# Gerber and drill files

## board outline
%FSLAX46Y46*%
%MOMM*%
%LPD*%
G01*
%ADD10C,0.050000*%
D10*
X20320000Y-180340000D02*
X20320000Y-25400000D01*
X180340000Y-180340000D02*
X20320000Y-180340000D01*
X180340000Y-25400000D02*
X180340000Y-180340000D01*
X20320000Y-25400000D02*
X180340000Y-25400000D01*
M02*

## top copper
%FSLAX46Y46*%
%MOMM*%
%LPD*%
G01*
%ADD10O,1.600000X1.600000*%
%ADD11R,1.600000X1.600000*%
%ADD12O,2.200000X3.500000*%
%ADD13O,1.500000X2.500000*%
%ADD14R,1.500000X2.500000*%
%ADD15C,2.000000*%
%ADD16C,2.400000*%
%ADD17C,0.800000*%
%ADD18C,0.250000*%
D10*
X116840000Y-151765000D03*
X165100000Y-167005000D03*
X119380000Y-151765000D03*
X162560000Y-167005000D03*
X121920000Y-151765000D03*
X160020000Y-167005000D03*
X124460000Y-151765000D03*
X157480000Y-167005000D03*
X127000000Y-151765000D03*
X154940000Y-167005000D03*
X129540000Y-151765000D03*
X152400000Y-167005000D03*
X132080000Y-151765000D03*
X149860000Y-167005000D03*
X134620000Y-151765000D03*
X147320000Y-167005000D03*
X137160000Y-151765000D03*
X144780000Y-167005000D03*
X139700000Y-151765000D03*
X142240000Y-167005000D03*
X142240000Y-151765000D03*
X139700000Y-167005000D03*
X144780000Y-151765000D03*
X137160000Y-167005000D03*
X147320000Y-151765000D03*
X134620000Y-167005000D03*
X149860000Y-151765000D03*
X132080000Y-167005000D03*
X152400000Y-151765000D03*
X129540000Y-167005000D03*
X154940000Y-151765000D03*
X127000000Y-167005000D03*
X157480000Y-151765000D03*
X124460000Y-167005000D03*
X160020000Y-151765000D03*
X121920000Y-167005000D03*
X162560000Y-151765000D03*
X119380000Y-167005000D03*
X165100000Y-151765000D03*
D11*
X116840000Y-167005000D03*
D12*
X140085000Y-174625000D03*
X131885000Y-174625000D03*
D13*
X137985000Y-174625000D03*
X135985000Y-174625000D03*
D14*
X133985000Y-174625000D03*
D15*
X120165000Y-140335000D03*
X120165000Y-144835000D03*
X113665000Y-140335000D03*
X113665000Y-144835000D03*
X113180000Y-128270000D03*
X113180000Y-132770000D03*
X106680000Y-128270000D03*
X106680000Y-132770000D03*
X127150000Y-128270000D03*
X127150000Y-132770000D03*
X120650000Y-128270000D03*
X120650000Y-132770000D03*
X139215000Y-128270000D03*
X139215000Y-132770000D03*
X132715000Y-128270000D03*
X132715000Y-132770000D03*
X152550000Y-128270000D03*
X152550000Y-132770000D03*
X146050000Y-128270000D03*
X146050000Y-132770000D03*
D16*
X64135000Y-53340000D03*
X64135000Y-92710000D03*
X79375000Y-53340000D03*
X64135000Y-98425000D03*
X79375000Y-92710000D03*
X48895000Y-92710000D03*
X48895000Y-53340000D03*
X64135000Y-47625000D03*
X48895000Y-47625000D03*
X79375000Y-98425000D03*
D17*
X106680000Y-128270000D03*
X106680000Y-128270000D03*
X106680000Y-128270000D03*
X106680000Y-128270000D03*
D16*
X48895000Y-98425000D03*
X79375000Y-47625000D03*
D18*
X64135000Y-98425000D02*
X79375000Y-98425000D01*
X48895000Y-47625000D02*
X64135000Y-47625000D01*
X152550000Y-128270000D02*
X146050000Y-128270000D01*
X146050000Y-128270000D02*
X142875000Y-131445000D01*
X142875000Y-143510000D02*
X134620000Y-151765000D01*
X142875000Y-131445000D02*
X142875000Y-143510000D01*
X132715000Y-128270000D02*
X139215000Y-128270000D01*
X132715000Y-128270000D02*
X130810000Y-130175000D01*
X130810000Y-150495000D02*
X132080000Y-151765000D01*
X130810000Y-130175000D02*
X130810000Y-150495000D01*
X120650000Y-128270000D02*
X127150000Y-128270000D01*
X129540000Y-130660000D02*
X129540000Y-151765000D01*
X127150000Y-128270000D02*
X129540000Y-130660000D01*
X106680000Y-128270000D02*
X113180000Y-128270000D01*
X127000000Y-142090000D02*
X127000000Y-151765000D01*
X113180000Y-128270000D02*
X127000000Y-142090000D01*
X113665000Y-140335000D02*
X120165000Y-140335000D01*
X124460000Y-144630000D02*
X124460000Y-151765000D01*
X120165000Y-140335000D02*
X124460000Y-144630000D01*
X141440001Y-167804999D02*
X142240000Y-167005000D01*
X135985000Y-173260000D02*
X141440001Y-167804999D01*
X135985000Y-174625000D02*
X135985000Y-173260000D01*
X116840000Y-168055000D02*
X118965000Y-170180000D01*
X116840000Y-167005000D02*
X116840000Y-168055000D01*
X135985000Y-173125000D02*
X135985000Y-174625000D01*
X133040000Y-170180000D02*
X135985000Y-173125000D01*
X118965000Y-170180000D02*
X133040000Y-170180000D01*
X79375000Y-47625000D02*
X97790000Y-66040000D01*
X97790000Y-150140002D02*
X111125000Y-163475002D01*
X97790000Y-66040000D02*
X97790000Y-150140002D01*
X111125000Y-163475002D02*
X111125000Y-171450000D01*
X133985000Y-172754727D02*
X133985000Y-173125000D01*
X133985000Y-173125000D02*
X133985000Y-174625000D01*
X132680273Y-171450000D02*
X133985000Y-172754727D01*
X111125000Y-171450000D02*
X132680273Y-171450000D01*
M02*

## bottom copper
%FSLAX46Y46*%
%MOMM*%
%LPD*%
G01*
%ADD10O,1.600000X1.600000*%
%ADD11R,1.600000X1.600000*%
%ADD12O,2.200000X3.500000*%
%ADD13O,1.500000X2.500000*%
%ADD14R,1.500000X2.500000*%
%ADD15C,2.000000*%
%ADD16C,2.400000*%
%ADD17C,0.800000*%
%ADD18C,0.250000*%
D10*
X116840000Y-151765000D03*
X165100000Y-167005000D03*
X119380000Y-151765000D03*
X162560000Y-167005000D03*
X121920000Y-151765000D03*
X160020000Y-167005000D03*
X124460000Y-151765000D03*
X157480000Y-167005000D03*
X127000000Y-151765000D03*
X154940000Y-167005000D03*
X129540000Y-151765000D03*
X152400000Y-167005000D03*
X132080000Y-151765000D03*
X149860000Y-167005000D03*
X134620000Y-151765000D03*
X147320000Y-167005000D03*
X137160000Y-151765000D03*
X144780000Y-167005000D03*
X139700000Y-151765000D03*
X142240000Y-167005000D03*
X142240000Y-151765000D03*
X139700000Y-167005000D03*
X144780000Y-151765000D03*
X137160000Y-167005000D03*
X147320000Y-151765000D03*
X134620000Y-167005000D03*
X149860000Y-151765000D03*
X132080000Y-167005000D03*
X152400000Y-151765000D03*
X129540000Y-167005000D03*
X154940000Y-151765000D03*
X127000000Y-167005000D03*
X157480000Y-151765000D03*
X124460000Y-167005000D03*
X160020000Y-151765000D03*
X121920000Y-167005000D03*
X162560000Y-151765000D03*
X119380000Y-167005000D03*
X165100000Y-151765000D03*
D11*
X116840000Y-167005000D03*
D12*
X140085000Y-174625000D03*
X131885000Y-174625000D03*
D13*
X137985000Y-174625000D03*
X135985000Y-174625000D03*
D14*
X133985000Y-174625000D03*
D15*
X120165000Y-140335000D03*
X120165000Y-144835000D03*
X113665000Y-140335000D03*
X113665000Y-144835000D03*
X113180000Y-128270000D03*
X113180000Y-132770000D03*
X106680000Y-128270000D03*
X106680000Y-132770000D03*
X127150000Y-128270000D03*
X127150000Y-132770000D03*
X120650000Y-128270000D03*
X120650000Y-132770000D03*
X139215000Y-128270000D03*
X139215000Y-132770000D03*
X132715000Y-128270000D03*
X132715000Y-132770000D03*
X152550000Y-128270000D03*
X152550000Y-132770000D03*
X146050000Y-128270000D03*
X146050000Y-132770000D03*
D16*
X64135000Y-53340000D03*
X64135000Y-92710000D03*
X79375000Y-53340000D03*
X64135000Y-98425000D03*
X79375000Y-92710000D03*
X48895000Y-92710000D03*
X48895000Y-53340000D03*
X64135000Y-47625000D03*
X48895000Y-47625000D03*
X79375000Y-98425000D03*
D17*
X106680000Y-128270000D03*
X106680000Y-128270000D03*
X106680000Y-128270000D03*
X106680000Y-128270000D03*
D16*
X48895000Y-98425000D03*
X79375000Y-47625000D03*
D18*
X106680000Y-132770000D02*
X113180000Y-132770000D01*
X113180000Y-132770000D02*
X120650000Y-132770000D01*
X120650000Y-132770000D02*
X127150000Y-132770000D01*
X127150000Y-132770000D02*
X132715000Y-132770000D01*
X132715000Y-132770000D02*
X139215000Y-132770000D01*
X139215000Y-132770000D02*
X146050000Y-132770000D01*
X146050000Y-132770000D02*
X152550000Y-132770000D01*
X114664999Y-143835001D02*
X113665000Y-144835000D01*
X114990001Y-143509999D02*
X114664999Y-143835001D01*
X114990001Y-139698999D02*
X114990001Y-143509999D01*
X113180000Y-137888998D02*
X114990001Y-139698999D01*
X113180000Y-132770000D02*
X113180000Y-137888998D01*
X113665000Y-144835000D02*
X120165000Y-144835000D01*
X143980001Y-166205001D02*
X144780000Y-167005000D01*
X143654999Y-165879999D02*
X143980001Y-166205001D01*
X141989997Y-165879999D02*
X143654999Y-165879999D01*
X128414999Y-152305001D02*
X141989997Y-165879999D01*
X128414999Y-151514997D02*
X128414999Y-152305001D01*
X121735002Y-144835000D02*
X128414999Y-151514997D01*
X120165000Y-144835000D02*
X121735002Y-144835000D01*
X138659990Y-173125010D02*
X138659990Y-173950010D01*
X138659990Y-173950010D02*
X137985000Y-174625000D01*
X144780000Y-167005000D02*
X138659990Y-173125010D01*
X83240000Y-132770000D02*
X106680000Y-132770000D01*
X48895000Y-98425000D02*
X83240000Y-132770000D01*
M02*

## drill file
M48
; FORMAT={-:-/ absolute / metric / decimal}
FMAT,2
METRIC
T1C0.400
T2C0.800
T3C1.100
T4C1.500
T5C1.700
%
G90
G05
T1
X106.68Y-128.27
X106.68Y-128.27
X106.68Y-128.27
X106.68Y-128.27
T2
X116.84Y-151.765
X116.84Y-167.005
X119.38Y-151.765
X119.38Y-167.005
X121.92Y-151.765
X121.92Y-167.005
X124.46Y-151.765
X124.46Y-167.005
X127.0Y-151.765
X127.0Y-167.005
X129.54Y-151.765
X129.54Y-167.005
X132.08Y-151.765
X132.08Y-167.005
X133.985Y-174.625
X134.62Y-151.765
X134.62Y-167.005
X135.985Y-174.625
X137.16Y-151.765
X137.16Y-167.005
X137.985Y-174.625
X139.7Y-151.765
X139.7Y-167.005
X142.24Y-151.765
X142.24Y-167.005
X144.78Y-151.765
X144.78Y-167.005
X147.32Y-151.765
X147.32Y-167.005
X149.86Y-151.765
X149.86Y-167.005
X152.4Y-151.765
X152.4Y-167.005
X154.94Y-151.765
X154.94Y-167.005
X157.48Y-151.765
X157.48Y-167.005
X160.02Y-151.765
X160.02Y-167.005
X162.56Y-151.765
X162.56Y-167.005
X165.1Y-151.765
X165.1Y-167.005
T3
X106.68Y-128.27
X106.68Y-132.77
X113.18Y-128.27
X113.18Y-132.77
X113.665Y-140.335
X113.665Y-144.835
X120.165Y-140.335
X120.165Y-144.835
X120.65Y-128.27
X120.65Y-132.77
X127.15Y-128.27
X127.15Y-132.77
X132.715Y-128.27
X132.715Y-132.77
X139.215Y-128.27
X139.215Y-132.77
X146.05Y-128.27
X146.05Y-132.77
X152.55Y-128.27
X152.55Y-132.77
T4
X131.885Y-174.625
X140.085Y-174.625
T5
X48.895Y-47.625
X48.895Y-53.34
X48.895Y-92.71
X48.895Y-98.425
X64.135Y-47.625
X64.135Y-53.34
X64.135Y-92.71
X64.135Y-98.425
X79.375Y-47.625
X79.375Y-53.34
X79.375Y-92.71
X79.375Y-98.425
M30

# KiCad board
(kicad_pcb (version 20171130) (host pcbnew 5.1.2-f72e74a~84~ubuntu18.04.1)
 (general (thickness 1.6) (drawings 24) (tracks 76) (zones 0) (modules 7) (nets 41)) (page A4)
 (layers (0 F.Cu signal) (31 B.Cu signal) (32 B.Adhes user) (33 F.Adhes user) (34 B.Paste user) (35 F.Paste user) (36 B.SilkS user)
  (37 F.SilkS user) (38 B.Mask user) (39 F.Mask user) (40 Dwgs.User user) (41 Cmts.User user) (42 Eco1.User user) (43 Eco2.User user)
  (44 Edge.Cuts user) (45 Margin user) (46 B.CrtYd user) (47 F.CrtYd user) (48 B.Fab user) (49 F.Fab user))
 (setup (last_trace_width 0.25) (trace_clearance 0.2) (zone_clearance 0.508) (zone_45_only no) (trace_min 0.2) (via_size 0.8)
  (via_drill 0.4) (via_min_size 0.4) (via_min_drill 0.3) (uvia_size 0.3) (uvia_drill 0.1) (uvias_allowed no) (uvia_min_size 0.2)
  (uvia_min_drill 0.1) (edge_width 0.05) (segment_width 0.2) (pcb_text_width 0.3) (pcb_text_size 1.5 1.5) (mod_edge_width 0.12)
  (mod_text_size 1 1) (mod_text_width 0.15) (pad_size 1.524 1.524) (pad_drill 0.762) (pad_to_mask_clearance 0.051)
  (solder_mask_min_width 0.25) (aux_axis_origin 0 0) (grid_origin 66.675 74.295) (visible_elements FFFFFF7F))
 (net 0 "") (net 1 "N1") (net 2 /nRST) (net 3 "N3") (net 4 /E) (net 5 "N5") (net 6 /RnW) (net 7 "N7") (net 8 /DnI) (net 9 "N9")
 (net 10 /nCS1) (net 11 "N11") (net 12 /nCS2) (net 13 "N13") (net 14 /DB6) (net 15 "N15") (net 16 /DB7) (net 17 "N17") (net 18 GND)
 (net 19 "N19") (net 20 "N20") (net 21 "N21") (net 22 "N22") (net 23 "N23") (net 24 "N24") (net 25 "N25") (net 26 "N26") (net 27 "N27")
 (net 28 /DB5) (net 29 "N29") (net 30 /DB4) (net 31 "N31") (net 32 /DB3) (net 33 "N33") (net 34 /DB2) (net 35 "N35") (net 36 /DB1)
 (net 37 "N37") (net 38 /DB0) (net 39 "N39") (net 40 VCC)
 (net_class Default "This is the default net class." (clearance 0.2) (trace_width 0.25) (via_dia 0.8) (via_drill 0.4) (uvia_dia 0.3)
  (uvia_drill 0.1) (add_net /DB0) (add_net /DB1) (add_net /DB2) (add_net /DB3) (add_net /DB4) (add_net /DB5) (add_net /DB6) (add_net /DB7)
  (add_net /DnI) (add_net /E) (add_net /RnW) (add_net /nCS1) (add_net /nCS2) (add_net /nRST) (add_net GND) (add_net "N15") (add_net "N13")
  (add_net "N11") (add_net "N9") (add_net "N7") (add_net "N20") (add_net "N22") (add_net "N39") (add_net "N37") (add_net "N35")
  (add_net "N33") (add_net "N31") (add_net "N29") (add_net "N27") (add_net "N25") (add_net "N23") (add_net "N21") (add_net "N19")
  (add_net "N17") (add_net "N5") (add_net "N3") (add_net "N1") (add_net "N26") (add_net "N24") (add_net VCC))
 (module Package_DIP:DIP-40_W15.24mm (layer F.Cu) (at 116.84 167.005 90)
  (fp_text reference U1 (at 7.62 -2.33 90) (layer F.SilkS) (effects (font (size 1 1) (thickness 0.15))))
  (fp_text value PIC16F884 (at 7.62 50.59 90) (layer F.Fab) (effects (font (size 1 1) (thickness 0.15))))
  (pad 40 thru_hole oval (at 15.24 0 90) (size 1.6 1.6) (drill 0.8) (layers *.Cu *.Mask) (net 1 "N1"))
  (pad 20 thru_hole oval (at 0 48.26 90) (size 1.6 1.6) (drill 0.8) (layers *.Cu *.Mask) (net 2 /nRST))
  (pad 39 thru_hole oval (at 15.24 2.54 90) (size 1.6 1.6) (drill 0.8) (layers *.Cu *.Mask) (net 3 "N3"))
  (pad 19 thru_hole oval (at 0 45.72 90) (size 1.6 1.6) (drill 0.8) (layers *.Cu *.Mask) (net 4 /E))
  (pad 38 thru_hole oval (at 15.24 5.08 90) (size 1.6 1.6) (drill 0.8) (layers *.Cu *.Mask) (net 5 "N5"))
  (pad 18 thru_hole oval (at 0 43.18 90) (size 1.6 1.6) (drill 0.8) (layers *.Cu *.Mask) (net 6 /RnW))
  (pad 37 thru_hole oval (at 15.24 7.62 90) (size 1.6 1.6) (drill 0.8) (layers *.Cu *.Mask) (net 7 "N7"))
  (pad 17 thru_hole oval (at 0 40.64 90) (size 1.6 1.6) (drill 0.8) (layers *.Cu *.Mask) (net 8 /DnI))
  (pad 36 thru_hole oval (at 15.24 10.16 90) (size 1.6 1.6) (drill 0.8) (layers *.Cu *.Mask) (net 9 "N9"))
  (pad 16 thru_hole oval (at 0 38.1 90) (size 1.6 1.6) (drill 0.8) (layers *.Cu *.Mask) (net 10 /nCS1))
  (pad 35 thru_hole oval (at 15.24 12.7 90) (size 1.6 1.6) (drill 0.8) (layers *.Cu *.Mask) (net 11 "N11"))
  (pad 15 thru_hole oval (at 0 35.56 90) (size 1.6 1.6) (drill 0.8) (layers *.Cu *.Mask) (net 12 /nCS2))
  (pad 34 thru_hole oval (at 15.24 15.24 90) (size 1.6 1.6) (drill 0.8) (layers *.Cu *.Mask) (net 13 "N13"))
  (pad 14 thru_hole oval (at 0 33.02 90) (size 1.6 1.6) (drill 0.8) (layers *.Cu *.Mask) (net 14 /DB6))
  (pad 33 thru_hole oval (at 15.24 17.78 90) (size 1.6 1.6) (drill 0.8) (layers *.Cu *.Mask) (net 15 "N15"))
  (pad 13 thru_hole oval (at 0 30.48 90) (size 1.6 1.6) (drill 0.8) (layers *.Cu *.Mask) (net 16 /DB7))
  (pad 32 thru_hole oval (at 15.24 20.32 90) (size 1.6 1.6) (drill 0.8) (layers *.Cu *.Mask) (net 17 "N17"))
  (pad 12 thru_hole oval (at 0 27.94 90) (size 1.6 1.6) (drill 0.8) (layers *.Cu *.Mask) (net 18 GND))
  (pad 31 thru_hole oval (at 15.24 22.86 90) (size 1.6 1.6) (drill 0.8) (layers *.Cu *.Mask) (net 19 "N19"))
  (pad 11 thru_hole oval (at 0 25.4 90) (size 1.6 1.6) (drill 0.8) (layers *.Cu *.Mask) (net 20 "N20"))
  (pad 30 thru_hole oval (at 15.24 25.4 90) (size 1.6 1.6) (drill 0.8) (layers *.Cu *.Mask) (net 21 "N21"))
  (pad 10 thru_hole oval (at 0 22.86 90) (size 1.6 1.6) (drill 0.8) (layers *.Cu *.Mask) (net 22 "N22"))
  (pad 29 thru_hole oval (at 15.24 27.94 90) (size 1.6 1.6) (drill 0.8) (layers *.Cu *.Mask) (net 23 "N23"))
  (pad 9 thru_hole oval (at 0 20.32 90) (size 1.6 1.6) (drill 0.8) (layers *.Cu *.Mask) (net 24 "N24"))
  (pad 28 thru_hole oval (at 15.24 30.48 90) (size 1.6 1.6) (drill 0.8) (layers *.Cu *.Mask) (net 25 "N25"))
  (pad 8 thru_hole oval (at 0 17.78 90) (size 1.6 1.6) (drill 0.8) (layers *.Cu *.Mask) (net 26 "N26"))
  (pad 27 thru_hole oval (at 15.24 33.02 90) (size 1.6 1.6) (drill 0.8) (layers *.Cu *.Mask) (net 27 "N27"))
  (pad 7 thru_hole oval (at 0 15.24 90) (size 1.6 1.6) (drill 0.8) (layers *.Cu *.Mask) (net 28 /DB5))
  (pad 26 thru_hole oval (at 15.24 35.56 90) (size 1.6 1.6) (drill 0.8) (layers *.Cu *.Mask) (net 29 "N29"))
  (pad 6 thru_hole oval (at 0 12.7 90) (size 1.6 1.6) (drill 0.8) (layers *.Cu *.Mask) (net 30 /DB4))
  (pad 25 thru_hole oval (at 15.24 38.1 90) (size 1.6 1.6) (drill 0.8) (layers *.Cu *.Mask) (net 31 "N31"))
  (pad 5 thru_hole oval (at 0 10.16 90) (size 1.6 1.6) (drill 0.8) (layers *.Cu *.Mask) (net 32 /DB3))
  (pad 24 thru_hole oval (at 15.24 40.64 90) (size 1.6 1.6) (drill 0.8) (layers *.Cu *.Mask) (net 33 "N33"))
  (pad 4 thru_hole oval (at 0 7.62 90) (size 1.6 1.6) (drill 0.8) (layers *.Cu *.Mask) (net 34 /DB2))
  (pad 23 thru_hole oval (at 15.24 43.18 90) (size 1.6 1.6) (drill 0.8) (layers *.Cu *.Mask) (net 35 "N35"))
  (pad 3 thru_hole oval (at 0 5.08 90) (size 1.6 1.6) (drill 0.8) (layers *.Cu *.Mask) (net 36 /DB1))
  (pad 22 thru_hole oval (at 15.24 45.72 90) (size 1.6 1.6) (drill 0.8) (layers *.Cu *.Mask) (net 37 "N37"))
  (pad 2 thru_hole oval (at 0 2.54 90) (size 1.6 1.6) (drill 0.8) (layers *.Cu *.Mask) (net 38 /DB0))
  (pad 21 thru_hole oval (at 15.24 48.26 90) (size 1.6 1.6) (drill 0.8) (layers *.Cu *.Mask) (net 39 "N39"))
  (pad 1 thru_hole rect (at 0 0 90) (size 1.6 1.6) (drill 0.8) (layers *.Cu *.Mask) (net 20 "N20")))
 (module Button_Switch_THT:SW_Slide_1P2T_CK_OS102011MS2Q (layer F.Cu) (at 133.985 174.625)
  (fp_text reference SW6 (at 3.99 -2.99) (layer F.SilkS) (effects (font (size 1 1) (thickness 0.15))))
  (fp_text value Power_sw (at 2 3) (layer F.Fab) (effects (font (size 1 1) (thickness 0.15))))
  (pad "" thru_hole oval (at 6.1 0) (size 2.2 3.5) (drill 1.5) (layers *.Cu *.Mask))
  (pad "" thru_hole oval (at -2.1 0) (size 2.2 3.5) (drill 1.5) (layers *.Cu *.Mask))
  (pad 3 thru_hole oval (at 4 0) (size 1.5 2.5) (drill 0.8) (layers *.Cu *.Mask) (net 18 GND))
  (pad 2 thru_hole oval (at 2 0) (size 1.5 2.5) (drill 0.8) (layers *.Cu *.Mask) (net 20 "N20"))
  (pad 1 thru_hole rect (at 0 0) (size 1.5 2.5) (drill 0.8) (layers *.Cu *.Mask) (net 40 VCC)))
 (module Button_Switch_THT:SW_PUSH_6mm (layer F.Cu) (at 113.665 140.335)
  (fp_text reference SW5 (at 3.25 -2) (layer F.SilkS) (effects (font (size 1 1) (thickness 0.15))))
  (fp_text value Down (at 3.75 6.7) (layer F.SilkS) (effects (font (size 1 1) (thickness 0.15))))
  (pad 1 thru_hole circle (at 6.5 0 90) (size 2 2) (drill 1.1) (layers *.Cu *.Mask) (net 7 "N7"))
  (pad 2 thru_hole circle (at 6.5 4.5 90) (size 2 2) (drill 1.1) (layers *.Cu *.Mask) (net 18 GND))
  (pad 1 thru_hole circle (at 0 0 90) (size 2 2) (drill 1.1) (layers *.Cu *.Mask) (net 7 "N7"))
  (pad 2 thru_hole circle (at 0 4.5 90) (size 2 2) (drill 1.1) (layers *.Cu *.Mask) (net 18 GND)))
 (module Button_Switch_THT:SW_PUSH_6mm (layer F.Cu) (at 106.68 128.27)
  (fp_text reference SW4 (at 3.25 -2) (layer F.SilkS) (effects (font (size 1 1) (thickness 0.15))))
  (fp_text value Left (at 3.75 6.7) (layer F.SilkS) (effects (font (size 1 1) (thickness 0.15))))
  (pad 1 thru_hole circle (at 6.5 0 90) (size 2 2) (drill 1.1) (layers *.Cu *.Mask) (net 9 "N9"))
  (pad 2 thru_hole circle (at 6.5 4.5 90) (size 2 2) (drill 1.1) (layers *.Cu *.Mask) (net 18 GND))
  (pad 1 thru_hole circle (at 0 0 90) (size 2 2) (drill 1.1) (layers *.Cu *.Mask) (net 9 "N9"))
  (pad 2 thru_hole circle (at 0 4.5 90) (size 2 2) (drill 1.1) (layers *.Cu *.Mask) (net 18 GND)))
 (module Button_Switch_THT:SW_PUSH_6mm (layer F.Cu) (at 120.65 128.27)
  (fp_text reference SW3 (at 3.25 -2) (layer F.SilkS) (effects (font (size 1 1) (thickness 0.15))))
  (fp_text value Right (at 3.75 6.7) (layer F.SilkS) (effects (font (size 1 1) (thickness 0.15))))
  (pad 1 thru_hole circle (at 6.5 0 90) (size 2 2) (drill 1.1) (layers *.Cu *.Mask) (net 11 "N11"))
  (pad 2 thru_hole circle (at 6.5 4.5 90) (size 2 2) (drill 1.1) (layers *.Cu *.Mask) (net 18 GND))
  (pad 1 thru_hole circle (at 0 0 90) (size 2 2) (drill 1.1) (layers *.Cu *.Mask) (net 11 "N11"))
  (pad 2 thru_hole circle (at 0 4.5 90) (size 2 2) (drill 1.1) (layers *.Cu *.Mask) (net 18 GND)))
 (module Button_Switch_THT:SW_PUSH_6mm (layer F.Cu) (at 132.715 128.27)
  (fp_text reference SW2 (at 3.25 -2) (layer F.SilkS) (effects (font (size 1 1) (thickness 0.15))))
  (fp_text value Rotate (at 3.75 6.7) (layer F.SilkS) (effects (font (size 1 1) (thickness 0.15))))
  (pad 1 thru_hole circle (at 6.5 0 90) (size 2 2) (drill 1.1) (layers *.Cu *.Mask) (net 13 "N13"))
  (pad 2 thru_hole circle (at 6.5 4.5 90) (size 2 2) (drill 1.1) (layers *.Cu *.Mask) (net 18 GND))
  (pad 1 thru_hole circle (at 0 0 90) (size 2 2) (drill 1.1) (layers *.Cu *.Mask) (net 13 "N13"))
  (pad 2 thru_hole circle (at 0 4.5 90) (size 2 2) (drill 1.1) (layers *.Cu *.Mask) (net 18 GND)))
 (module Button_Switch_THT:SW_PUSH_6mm (layer F.Cu) (at 146.05 128.27)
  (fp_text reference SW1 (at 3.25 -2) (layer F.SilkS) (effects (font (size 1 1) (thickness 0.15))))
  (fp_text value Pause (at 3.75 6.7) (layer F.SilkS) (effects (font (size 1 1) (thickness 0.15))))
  (pad 1 thru_hole circle (at 6.5 0 90) (size 2 2) (drill 1.1) (layers *.Cu *.Mask) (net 15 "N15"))
  (pad 2 thru_hole circle (at 6.5 4.5 90) (size 2 2) (drill 1.1) (layers *.Cu *.Mask) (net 18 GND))
  (pad 1 thru_hole circle (at 0 0 90) (size 2 2) (drill 1.1) (layers *.Cu *.Mask) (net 15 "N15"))
  (pad 2 thru_hole circle (at 0 4.5 90) (size 2 2) (drill 1.1) (layers *.Cu *.Mask) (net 18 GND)))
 (gr_line (start 20.32 180.34) (end 20.32 25.4) (layer Edge.Cuts) (width 0.05))
 (gr_line (start 180.34 180.34) (end 20.32 180.34) (layer Edge.Cuts) (width 0.05))
 (gr_line (start 180.34 25.4) (end 180.34 180.34) (layer Edge.Cuts) (width 0.05))
 (gr_line (start 20.32 25.4) (end 180.34 25.4) (layer Edge.Cuts) (width 0.05))
 (segment (start 64.135 98.425) (end 79.375 98.425) (width 0.25) (layer F.Cu) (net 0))
 (segment (start 48.895 47.625) (end 64.135 47.625) (width 0.25) (layer F.Cu) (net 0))
 (via (at 64.135 53.34) (size 2.4) (drill 1.7) (layers F.Cu B.Cu) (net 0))
 (via (at 64.135 92.71) (size 2.4) (drill 1.7) (layers F.Cu B.Cu) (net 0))
 (via (at 79.375 53.34) (size 2.4) (drill 1.7) (layers F.Cu B.Cu) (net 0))
 (via (at 64.135 98.425) (size 2.4) (drill 1.7) (layers F.Cu B.Cu) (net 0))
 (via (at 79.375 92.71) (size 2.4) (drill 1.7) (layers F.Cu B.Cu) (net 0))
 (via (at 48.895 92.71) (size 2.4) (drill 1.7) (layers F.Cu B.Cu) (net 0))
 (via (at 48.895 53.34) (size 2.4) (drill 1.7) (layers F.Cu B.Cu) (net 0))
 (via (at 64.135 47.625) (size 2.4) (drill 1.7) (layers F.Cu B.Cu) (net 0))
 (via (at 48.895 47.625) (size 2.4) (drill 1.7) (layers F.Cu B.Cu) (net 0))
 (via (at 79.375 98.425) (size 2.4) (drill 1.7) (layers F.Cu B.Cu) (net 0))
 (segment (start 152.55 128.27) (end 146.05 128.27) (width 0.25) (layer F.Cu) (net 15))
 (segment (start 146.05 128.27) (end 142.875 131.445) (width 0.25) (layer F.Cu) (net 15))
 (segment (start 142.875 143.51) (end 134.62 151.765) (width 0.25) (layer F.Cu) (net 15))
 (segment (start 142.875 131.445) (end 142.875 143.51) (width 0.25) (layer F.Cu) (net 15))
 (segment (start 132.715 128.27) (end 139.215 128.27) (width 0.25) (layer F.Cu) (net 13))
 (segment (start 132.715 128.27) (end 130.81 130.175) (width 0.25) (layer F.Cu) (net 13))
 (segment (start 130.81 150.495) (end 132.08 151.765) (width 0.25) (layer F.Cu) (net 13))
 (segment (start 130.81 130.175) (end 130.81 150.495) (width 0.25) (layer F.Cu) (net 13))
 (segment (start 120.65 128.27) (end 127.15 128.27) (width 0.25) (layer F.Cu) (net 11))
 (segment (start 129.54 130.66) (end 129.54 151.765) (width 0.25) (layer F.Cu) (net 11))
 (segment (start 127.15 128.27) (end 129.54 130.66) (width 0.25) (layer F.Cu) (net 11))
 (via (at 106.68 128.27) (size 0.8) (drill 0.4) (layers F.Cu B.Cu) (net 9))
 (via (at 106.68 128.27) (size 0.8) (drill 0.4) (layers F.Cu B.Cu) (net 9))
 (via (at 106.68 128.27) (size 0.8) (drill 0.4) (layers F.Cu B.Cu) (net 9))
 (via (at 106.68 128.27) (size 0.8) (drill 0.4) (layers F.Cu B.Cu) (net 9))
 (segment (start 106.68 128.27) (end 113.18 128.27) (width 0.25) (layer F.Cu) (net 9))
 (segment (start 127 142.09) (end 127 151.765) (width 0.25) (layer F.Cu) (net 9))
 (segment (start 113.18 128.27) (end 127 142.09) (width 0.25) (layer F.Cu) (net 9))
 (segment (start 113.665 140.335) (end 120.165 140.335) (width 0.25) (layer F.Cu) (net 7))
 (segment (start 124.46 144.63) (end 124.46 151.765) (width 0.25) (layer F.Cu) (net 7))
 (segment (start 120.165 140.335) (end 124.46 144.63) (width 0.25) (layer F.Cu) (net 7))
 (segment (start 106.68 132.77) (end 113.18 132.77) (width 0.25) (layer B.Cu) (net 18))
 (segment (start 113.18 132.77) (end 120.65 132.77) (width 0.25) (layer B.Cu) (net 18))
 (segment (start 120.65 132.77) (end 127.15 132.77) (width 0.25) (layer B.Cu) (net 18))
 (segment (start 127.15 132.77) (end 132.715 132.77) (width 0.25) (layer B.Cu) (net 18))
 (segment (start 132.715 132.77) (end 139.215 132.77) (width 0.25) (layer B.Cu) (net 18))
 (segment (start 139.215 132.77) (end 146.05 132.77) (width 0.25) (layer B.Cu) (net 18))
 (segment (start 146.05 132.77) (end 152.55 132.77) (width 0.25) (layer B.Cu) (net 18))
 (segment (start 114.664999 143.835001) (end 113.665 144.835) (width 0.25) (layer B.Cu) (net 18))
 (segment (start 114.990001 143.509999) (end 114.664999 143.835001) (width 0.25) (layer B.Cu) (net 18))
 (segment (start 114.990001 139.698999) (end 114.990001 143.509999) (width 0.25) (layer B.Cu) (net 18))
 (segment (start 113.18 137.888998) (end 114.990001 139.698999) (width 0.25) (layer B.Cu) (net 18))
 (segment (start 113.18 132.77) (end 113.18 137.888998) (width 0.25) (layer B.Cu) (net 18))
 (segment (start 113.665 144.835) (end 120.165 144.835) (width 0.25) (layer B.Cu) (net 18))
 (segment (start 143.980001 166.205001) (end 144.78 167.005) (width 0.25) (layer B.Cu) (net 18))
 (segment (start 143.654999 165.879999) (end 143.980001 166.205001) (width 0.25) (layer B.Cu) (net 18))
 (segment (start 141.989997 165.879999) (end 143.654999 165.879999) (width 0.25) (layer B.Cu) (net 18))
 (segment (start 128.414999 152.305001) (end 141.989997 165.879999) (width 0.25) (layer B.Cu) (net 18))
 (segment (start 128.414999 151.514997) (end 128.414999 152.305001) (width 0.25) (layer B.Cu) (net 18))
 (segment (start 121.735002 144.835) (end 128.414999 151.514997) (width 0.25) (layer B.Cu) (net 18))
 (segment (start 120.165 144.835) (end 121.735002 144.835) (width 0.25) (layer B.Cu) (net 18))
 (segment (start 138.65999 173.12501) (end 138.65999 173.95001) (width 0.25) (layer B.Cu) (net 18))
 (segment (start 138.65999 173.95001) (end 137.985 174.625) (width 0.25) (layer B.Cu) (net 18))
 (segment (start 144.78 167.005) (end 138.65999 173.12501) (width 0.25) (layer B.Cu) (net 18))
 (via (at 48.895 98.425) (size 2.4) (drill 1.7) (layers F.Cu B.Cu) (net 18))
 (segment (start 83.24 132.77) (end 106.68 132.77) (width 0.25) (layer B.Cu) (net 18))
 (segment (start 48.895 98.425) (end 83.24 132.77) (width 0.25) (layer B.Cu) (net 18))
 (segment (start 141.440001 167.804999) (end 142.24 167.005) (width 0.25) (layer F.Cu) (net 20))
 (segment (start 135.985 173.26) (end 141.440001 167.804999) (width 0.25) (layer F.Cu) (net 20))
 (segment (start 135.985 174.625) (end 135.985 173.26) (width 0.25) (layer F.Cu) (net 20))
 (segment (start 116.84 168.055) (end 118.965 170.18) (width 0.25) (layer F.Cu) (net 20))
 (segment (start 116.84 167.005) (end 116.84 168.055) (width 0.25) (layer F.Cu) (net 20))
 (segment (start 135.985 173.125) (end 135.985 174.625) (width 0.25) (layer F.Cu) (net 20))
 (segment (start 133.04 170.18) (end 135.985 173.125) (width 0.25) (layer F.Cu) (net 20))
 (segment (start 118.965 170.18) (end 133.04 170.18) (width 0.25) (layer F.Cu) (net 20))
 (via (at 79.375 47.625) (size 2.4) (drill 1.7) (layers F.Cu B.Cu) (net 40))
 (segment (start 79.375 47.625) (end 97.79 66.04) (width 0.25) (layer F.Cu) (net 40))
 (segment (start 97.79 150.140002) (end 111.125 163.475002) (width 0.25) (layer F.Cu) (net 40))
 (segment (start 97.79 66.04) (end 97.79 150.140002) (width 0.25) (layer F.Cu) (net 40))
 (segment (start 111.125 163.475002) (end 111.125 171.45) (width 0.25) (layer F.Cu) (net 40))
 (segment (start 133.985 172.754727) (end 133.985 173.125) (width 0.25) (layer F.Cu) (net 40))
 (segment (start 133.985 173.125) (end 133.985 174.625) (width 0.25) (layer F.Cu) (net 40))
 (segment (start 132.680273 171.45) (end 133.985 172.754727) (width 0.25) (layer F.Cu) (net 40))
 (segment (start 111.125 171.45) (end 132.680273 171.45) (width 0.25) (layer F.Cu) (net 40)))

